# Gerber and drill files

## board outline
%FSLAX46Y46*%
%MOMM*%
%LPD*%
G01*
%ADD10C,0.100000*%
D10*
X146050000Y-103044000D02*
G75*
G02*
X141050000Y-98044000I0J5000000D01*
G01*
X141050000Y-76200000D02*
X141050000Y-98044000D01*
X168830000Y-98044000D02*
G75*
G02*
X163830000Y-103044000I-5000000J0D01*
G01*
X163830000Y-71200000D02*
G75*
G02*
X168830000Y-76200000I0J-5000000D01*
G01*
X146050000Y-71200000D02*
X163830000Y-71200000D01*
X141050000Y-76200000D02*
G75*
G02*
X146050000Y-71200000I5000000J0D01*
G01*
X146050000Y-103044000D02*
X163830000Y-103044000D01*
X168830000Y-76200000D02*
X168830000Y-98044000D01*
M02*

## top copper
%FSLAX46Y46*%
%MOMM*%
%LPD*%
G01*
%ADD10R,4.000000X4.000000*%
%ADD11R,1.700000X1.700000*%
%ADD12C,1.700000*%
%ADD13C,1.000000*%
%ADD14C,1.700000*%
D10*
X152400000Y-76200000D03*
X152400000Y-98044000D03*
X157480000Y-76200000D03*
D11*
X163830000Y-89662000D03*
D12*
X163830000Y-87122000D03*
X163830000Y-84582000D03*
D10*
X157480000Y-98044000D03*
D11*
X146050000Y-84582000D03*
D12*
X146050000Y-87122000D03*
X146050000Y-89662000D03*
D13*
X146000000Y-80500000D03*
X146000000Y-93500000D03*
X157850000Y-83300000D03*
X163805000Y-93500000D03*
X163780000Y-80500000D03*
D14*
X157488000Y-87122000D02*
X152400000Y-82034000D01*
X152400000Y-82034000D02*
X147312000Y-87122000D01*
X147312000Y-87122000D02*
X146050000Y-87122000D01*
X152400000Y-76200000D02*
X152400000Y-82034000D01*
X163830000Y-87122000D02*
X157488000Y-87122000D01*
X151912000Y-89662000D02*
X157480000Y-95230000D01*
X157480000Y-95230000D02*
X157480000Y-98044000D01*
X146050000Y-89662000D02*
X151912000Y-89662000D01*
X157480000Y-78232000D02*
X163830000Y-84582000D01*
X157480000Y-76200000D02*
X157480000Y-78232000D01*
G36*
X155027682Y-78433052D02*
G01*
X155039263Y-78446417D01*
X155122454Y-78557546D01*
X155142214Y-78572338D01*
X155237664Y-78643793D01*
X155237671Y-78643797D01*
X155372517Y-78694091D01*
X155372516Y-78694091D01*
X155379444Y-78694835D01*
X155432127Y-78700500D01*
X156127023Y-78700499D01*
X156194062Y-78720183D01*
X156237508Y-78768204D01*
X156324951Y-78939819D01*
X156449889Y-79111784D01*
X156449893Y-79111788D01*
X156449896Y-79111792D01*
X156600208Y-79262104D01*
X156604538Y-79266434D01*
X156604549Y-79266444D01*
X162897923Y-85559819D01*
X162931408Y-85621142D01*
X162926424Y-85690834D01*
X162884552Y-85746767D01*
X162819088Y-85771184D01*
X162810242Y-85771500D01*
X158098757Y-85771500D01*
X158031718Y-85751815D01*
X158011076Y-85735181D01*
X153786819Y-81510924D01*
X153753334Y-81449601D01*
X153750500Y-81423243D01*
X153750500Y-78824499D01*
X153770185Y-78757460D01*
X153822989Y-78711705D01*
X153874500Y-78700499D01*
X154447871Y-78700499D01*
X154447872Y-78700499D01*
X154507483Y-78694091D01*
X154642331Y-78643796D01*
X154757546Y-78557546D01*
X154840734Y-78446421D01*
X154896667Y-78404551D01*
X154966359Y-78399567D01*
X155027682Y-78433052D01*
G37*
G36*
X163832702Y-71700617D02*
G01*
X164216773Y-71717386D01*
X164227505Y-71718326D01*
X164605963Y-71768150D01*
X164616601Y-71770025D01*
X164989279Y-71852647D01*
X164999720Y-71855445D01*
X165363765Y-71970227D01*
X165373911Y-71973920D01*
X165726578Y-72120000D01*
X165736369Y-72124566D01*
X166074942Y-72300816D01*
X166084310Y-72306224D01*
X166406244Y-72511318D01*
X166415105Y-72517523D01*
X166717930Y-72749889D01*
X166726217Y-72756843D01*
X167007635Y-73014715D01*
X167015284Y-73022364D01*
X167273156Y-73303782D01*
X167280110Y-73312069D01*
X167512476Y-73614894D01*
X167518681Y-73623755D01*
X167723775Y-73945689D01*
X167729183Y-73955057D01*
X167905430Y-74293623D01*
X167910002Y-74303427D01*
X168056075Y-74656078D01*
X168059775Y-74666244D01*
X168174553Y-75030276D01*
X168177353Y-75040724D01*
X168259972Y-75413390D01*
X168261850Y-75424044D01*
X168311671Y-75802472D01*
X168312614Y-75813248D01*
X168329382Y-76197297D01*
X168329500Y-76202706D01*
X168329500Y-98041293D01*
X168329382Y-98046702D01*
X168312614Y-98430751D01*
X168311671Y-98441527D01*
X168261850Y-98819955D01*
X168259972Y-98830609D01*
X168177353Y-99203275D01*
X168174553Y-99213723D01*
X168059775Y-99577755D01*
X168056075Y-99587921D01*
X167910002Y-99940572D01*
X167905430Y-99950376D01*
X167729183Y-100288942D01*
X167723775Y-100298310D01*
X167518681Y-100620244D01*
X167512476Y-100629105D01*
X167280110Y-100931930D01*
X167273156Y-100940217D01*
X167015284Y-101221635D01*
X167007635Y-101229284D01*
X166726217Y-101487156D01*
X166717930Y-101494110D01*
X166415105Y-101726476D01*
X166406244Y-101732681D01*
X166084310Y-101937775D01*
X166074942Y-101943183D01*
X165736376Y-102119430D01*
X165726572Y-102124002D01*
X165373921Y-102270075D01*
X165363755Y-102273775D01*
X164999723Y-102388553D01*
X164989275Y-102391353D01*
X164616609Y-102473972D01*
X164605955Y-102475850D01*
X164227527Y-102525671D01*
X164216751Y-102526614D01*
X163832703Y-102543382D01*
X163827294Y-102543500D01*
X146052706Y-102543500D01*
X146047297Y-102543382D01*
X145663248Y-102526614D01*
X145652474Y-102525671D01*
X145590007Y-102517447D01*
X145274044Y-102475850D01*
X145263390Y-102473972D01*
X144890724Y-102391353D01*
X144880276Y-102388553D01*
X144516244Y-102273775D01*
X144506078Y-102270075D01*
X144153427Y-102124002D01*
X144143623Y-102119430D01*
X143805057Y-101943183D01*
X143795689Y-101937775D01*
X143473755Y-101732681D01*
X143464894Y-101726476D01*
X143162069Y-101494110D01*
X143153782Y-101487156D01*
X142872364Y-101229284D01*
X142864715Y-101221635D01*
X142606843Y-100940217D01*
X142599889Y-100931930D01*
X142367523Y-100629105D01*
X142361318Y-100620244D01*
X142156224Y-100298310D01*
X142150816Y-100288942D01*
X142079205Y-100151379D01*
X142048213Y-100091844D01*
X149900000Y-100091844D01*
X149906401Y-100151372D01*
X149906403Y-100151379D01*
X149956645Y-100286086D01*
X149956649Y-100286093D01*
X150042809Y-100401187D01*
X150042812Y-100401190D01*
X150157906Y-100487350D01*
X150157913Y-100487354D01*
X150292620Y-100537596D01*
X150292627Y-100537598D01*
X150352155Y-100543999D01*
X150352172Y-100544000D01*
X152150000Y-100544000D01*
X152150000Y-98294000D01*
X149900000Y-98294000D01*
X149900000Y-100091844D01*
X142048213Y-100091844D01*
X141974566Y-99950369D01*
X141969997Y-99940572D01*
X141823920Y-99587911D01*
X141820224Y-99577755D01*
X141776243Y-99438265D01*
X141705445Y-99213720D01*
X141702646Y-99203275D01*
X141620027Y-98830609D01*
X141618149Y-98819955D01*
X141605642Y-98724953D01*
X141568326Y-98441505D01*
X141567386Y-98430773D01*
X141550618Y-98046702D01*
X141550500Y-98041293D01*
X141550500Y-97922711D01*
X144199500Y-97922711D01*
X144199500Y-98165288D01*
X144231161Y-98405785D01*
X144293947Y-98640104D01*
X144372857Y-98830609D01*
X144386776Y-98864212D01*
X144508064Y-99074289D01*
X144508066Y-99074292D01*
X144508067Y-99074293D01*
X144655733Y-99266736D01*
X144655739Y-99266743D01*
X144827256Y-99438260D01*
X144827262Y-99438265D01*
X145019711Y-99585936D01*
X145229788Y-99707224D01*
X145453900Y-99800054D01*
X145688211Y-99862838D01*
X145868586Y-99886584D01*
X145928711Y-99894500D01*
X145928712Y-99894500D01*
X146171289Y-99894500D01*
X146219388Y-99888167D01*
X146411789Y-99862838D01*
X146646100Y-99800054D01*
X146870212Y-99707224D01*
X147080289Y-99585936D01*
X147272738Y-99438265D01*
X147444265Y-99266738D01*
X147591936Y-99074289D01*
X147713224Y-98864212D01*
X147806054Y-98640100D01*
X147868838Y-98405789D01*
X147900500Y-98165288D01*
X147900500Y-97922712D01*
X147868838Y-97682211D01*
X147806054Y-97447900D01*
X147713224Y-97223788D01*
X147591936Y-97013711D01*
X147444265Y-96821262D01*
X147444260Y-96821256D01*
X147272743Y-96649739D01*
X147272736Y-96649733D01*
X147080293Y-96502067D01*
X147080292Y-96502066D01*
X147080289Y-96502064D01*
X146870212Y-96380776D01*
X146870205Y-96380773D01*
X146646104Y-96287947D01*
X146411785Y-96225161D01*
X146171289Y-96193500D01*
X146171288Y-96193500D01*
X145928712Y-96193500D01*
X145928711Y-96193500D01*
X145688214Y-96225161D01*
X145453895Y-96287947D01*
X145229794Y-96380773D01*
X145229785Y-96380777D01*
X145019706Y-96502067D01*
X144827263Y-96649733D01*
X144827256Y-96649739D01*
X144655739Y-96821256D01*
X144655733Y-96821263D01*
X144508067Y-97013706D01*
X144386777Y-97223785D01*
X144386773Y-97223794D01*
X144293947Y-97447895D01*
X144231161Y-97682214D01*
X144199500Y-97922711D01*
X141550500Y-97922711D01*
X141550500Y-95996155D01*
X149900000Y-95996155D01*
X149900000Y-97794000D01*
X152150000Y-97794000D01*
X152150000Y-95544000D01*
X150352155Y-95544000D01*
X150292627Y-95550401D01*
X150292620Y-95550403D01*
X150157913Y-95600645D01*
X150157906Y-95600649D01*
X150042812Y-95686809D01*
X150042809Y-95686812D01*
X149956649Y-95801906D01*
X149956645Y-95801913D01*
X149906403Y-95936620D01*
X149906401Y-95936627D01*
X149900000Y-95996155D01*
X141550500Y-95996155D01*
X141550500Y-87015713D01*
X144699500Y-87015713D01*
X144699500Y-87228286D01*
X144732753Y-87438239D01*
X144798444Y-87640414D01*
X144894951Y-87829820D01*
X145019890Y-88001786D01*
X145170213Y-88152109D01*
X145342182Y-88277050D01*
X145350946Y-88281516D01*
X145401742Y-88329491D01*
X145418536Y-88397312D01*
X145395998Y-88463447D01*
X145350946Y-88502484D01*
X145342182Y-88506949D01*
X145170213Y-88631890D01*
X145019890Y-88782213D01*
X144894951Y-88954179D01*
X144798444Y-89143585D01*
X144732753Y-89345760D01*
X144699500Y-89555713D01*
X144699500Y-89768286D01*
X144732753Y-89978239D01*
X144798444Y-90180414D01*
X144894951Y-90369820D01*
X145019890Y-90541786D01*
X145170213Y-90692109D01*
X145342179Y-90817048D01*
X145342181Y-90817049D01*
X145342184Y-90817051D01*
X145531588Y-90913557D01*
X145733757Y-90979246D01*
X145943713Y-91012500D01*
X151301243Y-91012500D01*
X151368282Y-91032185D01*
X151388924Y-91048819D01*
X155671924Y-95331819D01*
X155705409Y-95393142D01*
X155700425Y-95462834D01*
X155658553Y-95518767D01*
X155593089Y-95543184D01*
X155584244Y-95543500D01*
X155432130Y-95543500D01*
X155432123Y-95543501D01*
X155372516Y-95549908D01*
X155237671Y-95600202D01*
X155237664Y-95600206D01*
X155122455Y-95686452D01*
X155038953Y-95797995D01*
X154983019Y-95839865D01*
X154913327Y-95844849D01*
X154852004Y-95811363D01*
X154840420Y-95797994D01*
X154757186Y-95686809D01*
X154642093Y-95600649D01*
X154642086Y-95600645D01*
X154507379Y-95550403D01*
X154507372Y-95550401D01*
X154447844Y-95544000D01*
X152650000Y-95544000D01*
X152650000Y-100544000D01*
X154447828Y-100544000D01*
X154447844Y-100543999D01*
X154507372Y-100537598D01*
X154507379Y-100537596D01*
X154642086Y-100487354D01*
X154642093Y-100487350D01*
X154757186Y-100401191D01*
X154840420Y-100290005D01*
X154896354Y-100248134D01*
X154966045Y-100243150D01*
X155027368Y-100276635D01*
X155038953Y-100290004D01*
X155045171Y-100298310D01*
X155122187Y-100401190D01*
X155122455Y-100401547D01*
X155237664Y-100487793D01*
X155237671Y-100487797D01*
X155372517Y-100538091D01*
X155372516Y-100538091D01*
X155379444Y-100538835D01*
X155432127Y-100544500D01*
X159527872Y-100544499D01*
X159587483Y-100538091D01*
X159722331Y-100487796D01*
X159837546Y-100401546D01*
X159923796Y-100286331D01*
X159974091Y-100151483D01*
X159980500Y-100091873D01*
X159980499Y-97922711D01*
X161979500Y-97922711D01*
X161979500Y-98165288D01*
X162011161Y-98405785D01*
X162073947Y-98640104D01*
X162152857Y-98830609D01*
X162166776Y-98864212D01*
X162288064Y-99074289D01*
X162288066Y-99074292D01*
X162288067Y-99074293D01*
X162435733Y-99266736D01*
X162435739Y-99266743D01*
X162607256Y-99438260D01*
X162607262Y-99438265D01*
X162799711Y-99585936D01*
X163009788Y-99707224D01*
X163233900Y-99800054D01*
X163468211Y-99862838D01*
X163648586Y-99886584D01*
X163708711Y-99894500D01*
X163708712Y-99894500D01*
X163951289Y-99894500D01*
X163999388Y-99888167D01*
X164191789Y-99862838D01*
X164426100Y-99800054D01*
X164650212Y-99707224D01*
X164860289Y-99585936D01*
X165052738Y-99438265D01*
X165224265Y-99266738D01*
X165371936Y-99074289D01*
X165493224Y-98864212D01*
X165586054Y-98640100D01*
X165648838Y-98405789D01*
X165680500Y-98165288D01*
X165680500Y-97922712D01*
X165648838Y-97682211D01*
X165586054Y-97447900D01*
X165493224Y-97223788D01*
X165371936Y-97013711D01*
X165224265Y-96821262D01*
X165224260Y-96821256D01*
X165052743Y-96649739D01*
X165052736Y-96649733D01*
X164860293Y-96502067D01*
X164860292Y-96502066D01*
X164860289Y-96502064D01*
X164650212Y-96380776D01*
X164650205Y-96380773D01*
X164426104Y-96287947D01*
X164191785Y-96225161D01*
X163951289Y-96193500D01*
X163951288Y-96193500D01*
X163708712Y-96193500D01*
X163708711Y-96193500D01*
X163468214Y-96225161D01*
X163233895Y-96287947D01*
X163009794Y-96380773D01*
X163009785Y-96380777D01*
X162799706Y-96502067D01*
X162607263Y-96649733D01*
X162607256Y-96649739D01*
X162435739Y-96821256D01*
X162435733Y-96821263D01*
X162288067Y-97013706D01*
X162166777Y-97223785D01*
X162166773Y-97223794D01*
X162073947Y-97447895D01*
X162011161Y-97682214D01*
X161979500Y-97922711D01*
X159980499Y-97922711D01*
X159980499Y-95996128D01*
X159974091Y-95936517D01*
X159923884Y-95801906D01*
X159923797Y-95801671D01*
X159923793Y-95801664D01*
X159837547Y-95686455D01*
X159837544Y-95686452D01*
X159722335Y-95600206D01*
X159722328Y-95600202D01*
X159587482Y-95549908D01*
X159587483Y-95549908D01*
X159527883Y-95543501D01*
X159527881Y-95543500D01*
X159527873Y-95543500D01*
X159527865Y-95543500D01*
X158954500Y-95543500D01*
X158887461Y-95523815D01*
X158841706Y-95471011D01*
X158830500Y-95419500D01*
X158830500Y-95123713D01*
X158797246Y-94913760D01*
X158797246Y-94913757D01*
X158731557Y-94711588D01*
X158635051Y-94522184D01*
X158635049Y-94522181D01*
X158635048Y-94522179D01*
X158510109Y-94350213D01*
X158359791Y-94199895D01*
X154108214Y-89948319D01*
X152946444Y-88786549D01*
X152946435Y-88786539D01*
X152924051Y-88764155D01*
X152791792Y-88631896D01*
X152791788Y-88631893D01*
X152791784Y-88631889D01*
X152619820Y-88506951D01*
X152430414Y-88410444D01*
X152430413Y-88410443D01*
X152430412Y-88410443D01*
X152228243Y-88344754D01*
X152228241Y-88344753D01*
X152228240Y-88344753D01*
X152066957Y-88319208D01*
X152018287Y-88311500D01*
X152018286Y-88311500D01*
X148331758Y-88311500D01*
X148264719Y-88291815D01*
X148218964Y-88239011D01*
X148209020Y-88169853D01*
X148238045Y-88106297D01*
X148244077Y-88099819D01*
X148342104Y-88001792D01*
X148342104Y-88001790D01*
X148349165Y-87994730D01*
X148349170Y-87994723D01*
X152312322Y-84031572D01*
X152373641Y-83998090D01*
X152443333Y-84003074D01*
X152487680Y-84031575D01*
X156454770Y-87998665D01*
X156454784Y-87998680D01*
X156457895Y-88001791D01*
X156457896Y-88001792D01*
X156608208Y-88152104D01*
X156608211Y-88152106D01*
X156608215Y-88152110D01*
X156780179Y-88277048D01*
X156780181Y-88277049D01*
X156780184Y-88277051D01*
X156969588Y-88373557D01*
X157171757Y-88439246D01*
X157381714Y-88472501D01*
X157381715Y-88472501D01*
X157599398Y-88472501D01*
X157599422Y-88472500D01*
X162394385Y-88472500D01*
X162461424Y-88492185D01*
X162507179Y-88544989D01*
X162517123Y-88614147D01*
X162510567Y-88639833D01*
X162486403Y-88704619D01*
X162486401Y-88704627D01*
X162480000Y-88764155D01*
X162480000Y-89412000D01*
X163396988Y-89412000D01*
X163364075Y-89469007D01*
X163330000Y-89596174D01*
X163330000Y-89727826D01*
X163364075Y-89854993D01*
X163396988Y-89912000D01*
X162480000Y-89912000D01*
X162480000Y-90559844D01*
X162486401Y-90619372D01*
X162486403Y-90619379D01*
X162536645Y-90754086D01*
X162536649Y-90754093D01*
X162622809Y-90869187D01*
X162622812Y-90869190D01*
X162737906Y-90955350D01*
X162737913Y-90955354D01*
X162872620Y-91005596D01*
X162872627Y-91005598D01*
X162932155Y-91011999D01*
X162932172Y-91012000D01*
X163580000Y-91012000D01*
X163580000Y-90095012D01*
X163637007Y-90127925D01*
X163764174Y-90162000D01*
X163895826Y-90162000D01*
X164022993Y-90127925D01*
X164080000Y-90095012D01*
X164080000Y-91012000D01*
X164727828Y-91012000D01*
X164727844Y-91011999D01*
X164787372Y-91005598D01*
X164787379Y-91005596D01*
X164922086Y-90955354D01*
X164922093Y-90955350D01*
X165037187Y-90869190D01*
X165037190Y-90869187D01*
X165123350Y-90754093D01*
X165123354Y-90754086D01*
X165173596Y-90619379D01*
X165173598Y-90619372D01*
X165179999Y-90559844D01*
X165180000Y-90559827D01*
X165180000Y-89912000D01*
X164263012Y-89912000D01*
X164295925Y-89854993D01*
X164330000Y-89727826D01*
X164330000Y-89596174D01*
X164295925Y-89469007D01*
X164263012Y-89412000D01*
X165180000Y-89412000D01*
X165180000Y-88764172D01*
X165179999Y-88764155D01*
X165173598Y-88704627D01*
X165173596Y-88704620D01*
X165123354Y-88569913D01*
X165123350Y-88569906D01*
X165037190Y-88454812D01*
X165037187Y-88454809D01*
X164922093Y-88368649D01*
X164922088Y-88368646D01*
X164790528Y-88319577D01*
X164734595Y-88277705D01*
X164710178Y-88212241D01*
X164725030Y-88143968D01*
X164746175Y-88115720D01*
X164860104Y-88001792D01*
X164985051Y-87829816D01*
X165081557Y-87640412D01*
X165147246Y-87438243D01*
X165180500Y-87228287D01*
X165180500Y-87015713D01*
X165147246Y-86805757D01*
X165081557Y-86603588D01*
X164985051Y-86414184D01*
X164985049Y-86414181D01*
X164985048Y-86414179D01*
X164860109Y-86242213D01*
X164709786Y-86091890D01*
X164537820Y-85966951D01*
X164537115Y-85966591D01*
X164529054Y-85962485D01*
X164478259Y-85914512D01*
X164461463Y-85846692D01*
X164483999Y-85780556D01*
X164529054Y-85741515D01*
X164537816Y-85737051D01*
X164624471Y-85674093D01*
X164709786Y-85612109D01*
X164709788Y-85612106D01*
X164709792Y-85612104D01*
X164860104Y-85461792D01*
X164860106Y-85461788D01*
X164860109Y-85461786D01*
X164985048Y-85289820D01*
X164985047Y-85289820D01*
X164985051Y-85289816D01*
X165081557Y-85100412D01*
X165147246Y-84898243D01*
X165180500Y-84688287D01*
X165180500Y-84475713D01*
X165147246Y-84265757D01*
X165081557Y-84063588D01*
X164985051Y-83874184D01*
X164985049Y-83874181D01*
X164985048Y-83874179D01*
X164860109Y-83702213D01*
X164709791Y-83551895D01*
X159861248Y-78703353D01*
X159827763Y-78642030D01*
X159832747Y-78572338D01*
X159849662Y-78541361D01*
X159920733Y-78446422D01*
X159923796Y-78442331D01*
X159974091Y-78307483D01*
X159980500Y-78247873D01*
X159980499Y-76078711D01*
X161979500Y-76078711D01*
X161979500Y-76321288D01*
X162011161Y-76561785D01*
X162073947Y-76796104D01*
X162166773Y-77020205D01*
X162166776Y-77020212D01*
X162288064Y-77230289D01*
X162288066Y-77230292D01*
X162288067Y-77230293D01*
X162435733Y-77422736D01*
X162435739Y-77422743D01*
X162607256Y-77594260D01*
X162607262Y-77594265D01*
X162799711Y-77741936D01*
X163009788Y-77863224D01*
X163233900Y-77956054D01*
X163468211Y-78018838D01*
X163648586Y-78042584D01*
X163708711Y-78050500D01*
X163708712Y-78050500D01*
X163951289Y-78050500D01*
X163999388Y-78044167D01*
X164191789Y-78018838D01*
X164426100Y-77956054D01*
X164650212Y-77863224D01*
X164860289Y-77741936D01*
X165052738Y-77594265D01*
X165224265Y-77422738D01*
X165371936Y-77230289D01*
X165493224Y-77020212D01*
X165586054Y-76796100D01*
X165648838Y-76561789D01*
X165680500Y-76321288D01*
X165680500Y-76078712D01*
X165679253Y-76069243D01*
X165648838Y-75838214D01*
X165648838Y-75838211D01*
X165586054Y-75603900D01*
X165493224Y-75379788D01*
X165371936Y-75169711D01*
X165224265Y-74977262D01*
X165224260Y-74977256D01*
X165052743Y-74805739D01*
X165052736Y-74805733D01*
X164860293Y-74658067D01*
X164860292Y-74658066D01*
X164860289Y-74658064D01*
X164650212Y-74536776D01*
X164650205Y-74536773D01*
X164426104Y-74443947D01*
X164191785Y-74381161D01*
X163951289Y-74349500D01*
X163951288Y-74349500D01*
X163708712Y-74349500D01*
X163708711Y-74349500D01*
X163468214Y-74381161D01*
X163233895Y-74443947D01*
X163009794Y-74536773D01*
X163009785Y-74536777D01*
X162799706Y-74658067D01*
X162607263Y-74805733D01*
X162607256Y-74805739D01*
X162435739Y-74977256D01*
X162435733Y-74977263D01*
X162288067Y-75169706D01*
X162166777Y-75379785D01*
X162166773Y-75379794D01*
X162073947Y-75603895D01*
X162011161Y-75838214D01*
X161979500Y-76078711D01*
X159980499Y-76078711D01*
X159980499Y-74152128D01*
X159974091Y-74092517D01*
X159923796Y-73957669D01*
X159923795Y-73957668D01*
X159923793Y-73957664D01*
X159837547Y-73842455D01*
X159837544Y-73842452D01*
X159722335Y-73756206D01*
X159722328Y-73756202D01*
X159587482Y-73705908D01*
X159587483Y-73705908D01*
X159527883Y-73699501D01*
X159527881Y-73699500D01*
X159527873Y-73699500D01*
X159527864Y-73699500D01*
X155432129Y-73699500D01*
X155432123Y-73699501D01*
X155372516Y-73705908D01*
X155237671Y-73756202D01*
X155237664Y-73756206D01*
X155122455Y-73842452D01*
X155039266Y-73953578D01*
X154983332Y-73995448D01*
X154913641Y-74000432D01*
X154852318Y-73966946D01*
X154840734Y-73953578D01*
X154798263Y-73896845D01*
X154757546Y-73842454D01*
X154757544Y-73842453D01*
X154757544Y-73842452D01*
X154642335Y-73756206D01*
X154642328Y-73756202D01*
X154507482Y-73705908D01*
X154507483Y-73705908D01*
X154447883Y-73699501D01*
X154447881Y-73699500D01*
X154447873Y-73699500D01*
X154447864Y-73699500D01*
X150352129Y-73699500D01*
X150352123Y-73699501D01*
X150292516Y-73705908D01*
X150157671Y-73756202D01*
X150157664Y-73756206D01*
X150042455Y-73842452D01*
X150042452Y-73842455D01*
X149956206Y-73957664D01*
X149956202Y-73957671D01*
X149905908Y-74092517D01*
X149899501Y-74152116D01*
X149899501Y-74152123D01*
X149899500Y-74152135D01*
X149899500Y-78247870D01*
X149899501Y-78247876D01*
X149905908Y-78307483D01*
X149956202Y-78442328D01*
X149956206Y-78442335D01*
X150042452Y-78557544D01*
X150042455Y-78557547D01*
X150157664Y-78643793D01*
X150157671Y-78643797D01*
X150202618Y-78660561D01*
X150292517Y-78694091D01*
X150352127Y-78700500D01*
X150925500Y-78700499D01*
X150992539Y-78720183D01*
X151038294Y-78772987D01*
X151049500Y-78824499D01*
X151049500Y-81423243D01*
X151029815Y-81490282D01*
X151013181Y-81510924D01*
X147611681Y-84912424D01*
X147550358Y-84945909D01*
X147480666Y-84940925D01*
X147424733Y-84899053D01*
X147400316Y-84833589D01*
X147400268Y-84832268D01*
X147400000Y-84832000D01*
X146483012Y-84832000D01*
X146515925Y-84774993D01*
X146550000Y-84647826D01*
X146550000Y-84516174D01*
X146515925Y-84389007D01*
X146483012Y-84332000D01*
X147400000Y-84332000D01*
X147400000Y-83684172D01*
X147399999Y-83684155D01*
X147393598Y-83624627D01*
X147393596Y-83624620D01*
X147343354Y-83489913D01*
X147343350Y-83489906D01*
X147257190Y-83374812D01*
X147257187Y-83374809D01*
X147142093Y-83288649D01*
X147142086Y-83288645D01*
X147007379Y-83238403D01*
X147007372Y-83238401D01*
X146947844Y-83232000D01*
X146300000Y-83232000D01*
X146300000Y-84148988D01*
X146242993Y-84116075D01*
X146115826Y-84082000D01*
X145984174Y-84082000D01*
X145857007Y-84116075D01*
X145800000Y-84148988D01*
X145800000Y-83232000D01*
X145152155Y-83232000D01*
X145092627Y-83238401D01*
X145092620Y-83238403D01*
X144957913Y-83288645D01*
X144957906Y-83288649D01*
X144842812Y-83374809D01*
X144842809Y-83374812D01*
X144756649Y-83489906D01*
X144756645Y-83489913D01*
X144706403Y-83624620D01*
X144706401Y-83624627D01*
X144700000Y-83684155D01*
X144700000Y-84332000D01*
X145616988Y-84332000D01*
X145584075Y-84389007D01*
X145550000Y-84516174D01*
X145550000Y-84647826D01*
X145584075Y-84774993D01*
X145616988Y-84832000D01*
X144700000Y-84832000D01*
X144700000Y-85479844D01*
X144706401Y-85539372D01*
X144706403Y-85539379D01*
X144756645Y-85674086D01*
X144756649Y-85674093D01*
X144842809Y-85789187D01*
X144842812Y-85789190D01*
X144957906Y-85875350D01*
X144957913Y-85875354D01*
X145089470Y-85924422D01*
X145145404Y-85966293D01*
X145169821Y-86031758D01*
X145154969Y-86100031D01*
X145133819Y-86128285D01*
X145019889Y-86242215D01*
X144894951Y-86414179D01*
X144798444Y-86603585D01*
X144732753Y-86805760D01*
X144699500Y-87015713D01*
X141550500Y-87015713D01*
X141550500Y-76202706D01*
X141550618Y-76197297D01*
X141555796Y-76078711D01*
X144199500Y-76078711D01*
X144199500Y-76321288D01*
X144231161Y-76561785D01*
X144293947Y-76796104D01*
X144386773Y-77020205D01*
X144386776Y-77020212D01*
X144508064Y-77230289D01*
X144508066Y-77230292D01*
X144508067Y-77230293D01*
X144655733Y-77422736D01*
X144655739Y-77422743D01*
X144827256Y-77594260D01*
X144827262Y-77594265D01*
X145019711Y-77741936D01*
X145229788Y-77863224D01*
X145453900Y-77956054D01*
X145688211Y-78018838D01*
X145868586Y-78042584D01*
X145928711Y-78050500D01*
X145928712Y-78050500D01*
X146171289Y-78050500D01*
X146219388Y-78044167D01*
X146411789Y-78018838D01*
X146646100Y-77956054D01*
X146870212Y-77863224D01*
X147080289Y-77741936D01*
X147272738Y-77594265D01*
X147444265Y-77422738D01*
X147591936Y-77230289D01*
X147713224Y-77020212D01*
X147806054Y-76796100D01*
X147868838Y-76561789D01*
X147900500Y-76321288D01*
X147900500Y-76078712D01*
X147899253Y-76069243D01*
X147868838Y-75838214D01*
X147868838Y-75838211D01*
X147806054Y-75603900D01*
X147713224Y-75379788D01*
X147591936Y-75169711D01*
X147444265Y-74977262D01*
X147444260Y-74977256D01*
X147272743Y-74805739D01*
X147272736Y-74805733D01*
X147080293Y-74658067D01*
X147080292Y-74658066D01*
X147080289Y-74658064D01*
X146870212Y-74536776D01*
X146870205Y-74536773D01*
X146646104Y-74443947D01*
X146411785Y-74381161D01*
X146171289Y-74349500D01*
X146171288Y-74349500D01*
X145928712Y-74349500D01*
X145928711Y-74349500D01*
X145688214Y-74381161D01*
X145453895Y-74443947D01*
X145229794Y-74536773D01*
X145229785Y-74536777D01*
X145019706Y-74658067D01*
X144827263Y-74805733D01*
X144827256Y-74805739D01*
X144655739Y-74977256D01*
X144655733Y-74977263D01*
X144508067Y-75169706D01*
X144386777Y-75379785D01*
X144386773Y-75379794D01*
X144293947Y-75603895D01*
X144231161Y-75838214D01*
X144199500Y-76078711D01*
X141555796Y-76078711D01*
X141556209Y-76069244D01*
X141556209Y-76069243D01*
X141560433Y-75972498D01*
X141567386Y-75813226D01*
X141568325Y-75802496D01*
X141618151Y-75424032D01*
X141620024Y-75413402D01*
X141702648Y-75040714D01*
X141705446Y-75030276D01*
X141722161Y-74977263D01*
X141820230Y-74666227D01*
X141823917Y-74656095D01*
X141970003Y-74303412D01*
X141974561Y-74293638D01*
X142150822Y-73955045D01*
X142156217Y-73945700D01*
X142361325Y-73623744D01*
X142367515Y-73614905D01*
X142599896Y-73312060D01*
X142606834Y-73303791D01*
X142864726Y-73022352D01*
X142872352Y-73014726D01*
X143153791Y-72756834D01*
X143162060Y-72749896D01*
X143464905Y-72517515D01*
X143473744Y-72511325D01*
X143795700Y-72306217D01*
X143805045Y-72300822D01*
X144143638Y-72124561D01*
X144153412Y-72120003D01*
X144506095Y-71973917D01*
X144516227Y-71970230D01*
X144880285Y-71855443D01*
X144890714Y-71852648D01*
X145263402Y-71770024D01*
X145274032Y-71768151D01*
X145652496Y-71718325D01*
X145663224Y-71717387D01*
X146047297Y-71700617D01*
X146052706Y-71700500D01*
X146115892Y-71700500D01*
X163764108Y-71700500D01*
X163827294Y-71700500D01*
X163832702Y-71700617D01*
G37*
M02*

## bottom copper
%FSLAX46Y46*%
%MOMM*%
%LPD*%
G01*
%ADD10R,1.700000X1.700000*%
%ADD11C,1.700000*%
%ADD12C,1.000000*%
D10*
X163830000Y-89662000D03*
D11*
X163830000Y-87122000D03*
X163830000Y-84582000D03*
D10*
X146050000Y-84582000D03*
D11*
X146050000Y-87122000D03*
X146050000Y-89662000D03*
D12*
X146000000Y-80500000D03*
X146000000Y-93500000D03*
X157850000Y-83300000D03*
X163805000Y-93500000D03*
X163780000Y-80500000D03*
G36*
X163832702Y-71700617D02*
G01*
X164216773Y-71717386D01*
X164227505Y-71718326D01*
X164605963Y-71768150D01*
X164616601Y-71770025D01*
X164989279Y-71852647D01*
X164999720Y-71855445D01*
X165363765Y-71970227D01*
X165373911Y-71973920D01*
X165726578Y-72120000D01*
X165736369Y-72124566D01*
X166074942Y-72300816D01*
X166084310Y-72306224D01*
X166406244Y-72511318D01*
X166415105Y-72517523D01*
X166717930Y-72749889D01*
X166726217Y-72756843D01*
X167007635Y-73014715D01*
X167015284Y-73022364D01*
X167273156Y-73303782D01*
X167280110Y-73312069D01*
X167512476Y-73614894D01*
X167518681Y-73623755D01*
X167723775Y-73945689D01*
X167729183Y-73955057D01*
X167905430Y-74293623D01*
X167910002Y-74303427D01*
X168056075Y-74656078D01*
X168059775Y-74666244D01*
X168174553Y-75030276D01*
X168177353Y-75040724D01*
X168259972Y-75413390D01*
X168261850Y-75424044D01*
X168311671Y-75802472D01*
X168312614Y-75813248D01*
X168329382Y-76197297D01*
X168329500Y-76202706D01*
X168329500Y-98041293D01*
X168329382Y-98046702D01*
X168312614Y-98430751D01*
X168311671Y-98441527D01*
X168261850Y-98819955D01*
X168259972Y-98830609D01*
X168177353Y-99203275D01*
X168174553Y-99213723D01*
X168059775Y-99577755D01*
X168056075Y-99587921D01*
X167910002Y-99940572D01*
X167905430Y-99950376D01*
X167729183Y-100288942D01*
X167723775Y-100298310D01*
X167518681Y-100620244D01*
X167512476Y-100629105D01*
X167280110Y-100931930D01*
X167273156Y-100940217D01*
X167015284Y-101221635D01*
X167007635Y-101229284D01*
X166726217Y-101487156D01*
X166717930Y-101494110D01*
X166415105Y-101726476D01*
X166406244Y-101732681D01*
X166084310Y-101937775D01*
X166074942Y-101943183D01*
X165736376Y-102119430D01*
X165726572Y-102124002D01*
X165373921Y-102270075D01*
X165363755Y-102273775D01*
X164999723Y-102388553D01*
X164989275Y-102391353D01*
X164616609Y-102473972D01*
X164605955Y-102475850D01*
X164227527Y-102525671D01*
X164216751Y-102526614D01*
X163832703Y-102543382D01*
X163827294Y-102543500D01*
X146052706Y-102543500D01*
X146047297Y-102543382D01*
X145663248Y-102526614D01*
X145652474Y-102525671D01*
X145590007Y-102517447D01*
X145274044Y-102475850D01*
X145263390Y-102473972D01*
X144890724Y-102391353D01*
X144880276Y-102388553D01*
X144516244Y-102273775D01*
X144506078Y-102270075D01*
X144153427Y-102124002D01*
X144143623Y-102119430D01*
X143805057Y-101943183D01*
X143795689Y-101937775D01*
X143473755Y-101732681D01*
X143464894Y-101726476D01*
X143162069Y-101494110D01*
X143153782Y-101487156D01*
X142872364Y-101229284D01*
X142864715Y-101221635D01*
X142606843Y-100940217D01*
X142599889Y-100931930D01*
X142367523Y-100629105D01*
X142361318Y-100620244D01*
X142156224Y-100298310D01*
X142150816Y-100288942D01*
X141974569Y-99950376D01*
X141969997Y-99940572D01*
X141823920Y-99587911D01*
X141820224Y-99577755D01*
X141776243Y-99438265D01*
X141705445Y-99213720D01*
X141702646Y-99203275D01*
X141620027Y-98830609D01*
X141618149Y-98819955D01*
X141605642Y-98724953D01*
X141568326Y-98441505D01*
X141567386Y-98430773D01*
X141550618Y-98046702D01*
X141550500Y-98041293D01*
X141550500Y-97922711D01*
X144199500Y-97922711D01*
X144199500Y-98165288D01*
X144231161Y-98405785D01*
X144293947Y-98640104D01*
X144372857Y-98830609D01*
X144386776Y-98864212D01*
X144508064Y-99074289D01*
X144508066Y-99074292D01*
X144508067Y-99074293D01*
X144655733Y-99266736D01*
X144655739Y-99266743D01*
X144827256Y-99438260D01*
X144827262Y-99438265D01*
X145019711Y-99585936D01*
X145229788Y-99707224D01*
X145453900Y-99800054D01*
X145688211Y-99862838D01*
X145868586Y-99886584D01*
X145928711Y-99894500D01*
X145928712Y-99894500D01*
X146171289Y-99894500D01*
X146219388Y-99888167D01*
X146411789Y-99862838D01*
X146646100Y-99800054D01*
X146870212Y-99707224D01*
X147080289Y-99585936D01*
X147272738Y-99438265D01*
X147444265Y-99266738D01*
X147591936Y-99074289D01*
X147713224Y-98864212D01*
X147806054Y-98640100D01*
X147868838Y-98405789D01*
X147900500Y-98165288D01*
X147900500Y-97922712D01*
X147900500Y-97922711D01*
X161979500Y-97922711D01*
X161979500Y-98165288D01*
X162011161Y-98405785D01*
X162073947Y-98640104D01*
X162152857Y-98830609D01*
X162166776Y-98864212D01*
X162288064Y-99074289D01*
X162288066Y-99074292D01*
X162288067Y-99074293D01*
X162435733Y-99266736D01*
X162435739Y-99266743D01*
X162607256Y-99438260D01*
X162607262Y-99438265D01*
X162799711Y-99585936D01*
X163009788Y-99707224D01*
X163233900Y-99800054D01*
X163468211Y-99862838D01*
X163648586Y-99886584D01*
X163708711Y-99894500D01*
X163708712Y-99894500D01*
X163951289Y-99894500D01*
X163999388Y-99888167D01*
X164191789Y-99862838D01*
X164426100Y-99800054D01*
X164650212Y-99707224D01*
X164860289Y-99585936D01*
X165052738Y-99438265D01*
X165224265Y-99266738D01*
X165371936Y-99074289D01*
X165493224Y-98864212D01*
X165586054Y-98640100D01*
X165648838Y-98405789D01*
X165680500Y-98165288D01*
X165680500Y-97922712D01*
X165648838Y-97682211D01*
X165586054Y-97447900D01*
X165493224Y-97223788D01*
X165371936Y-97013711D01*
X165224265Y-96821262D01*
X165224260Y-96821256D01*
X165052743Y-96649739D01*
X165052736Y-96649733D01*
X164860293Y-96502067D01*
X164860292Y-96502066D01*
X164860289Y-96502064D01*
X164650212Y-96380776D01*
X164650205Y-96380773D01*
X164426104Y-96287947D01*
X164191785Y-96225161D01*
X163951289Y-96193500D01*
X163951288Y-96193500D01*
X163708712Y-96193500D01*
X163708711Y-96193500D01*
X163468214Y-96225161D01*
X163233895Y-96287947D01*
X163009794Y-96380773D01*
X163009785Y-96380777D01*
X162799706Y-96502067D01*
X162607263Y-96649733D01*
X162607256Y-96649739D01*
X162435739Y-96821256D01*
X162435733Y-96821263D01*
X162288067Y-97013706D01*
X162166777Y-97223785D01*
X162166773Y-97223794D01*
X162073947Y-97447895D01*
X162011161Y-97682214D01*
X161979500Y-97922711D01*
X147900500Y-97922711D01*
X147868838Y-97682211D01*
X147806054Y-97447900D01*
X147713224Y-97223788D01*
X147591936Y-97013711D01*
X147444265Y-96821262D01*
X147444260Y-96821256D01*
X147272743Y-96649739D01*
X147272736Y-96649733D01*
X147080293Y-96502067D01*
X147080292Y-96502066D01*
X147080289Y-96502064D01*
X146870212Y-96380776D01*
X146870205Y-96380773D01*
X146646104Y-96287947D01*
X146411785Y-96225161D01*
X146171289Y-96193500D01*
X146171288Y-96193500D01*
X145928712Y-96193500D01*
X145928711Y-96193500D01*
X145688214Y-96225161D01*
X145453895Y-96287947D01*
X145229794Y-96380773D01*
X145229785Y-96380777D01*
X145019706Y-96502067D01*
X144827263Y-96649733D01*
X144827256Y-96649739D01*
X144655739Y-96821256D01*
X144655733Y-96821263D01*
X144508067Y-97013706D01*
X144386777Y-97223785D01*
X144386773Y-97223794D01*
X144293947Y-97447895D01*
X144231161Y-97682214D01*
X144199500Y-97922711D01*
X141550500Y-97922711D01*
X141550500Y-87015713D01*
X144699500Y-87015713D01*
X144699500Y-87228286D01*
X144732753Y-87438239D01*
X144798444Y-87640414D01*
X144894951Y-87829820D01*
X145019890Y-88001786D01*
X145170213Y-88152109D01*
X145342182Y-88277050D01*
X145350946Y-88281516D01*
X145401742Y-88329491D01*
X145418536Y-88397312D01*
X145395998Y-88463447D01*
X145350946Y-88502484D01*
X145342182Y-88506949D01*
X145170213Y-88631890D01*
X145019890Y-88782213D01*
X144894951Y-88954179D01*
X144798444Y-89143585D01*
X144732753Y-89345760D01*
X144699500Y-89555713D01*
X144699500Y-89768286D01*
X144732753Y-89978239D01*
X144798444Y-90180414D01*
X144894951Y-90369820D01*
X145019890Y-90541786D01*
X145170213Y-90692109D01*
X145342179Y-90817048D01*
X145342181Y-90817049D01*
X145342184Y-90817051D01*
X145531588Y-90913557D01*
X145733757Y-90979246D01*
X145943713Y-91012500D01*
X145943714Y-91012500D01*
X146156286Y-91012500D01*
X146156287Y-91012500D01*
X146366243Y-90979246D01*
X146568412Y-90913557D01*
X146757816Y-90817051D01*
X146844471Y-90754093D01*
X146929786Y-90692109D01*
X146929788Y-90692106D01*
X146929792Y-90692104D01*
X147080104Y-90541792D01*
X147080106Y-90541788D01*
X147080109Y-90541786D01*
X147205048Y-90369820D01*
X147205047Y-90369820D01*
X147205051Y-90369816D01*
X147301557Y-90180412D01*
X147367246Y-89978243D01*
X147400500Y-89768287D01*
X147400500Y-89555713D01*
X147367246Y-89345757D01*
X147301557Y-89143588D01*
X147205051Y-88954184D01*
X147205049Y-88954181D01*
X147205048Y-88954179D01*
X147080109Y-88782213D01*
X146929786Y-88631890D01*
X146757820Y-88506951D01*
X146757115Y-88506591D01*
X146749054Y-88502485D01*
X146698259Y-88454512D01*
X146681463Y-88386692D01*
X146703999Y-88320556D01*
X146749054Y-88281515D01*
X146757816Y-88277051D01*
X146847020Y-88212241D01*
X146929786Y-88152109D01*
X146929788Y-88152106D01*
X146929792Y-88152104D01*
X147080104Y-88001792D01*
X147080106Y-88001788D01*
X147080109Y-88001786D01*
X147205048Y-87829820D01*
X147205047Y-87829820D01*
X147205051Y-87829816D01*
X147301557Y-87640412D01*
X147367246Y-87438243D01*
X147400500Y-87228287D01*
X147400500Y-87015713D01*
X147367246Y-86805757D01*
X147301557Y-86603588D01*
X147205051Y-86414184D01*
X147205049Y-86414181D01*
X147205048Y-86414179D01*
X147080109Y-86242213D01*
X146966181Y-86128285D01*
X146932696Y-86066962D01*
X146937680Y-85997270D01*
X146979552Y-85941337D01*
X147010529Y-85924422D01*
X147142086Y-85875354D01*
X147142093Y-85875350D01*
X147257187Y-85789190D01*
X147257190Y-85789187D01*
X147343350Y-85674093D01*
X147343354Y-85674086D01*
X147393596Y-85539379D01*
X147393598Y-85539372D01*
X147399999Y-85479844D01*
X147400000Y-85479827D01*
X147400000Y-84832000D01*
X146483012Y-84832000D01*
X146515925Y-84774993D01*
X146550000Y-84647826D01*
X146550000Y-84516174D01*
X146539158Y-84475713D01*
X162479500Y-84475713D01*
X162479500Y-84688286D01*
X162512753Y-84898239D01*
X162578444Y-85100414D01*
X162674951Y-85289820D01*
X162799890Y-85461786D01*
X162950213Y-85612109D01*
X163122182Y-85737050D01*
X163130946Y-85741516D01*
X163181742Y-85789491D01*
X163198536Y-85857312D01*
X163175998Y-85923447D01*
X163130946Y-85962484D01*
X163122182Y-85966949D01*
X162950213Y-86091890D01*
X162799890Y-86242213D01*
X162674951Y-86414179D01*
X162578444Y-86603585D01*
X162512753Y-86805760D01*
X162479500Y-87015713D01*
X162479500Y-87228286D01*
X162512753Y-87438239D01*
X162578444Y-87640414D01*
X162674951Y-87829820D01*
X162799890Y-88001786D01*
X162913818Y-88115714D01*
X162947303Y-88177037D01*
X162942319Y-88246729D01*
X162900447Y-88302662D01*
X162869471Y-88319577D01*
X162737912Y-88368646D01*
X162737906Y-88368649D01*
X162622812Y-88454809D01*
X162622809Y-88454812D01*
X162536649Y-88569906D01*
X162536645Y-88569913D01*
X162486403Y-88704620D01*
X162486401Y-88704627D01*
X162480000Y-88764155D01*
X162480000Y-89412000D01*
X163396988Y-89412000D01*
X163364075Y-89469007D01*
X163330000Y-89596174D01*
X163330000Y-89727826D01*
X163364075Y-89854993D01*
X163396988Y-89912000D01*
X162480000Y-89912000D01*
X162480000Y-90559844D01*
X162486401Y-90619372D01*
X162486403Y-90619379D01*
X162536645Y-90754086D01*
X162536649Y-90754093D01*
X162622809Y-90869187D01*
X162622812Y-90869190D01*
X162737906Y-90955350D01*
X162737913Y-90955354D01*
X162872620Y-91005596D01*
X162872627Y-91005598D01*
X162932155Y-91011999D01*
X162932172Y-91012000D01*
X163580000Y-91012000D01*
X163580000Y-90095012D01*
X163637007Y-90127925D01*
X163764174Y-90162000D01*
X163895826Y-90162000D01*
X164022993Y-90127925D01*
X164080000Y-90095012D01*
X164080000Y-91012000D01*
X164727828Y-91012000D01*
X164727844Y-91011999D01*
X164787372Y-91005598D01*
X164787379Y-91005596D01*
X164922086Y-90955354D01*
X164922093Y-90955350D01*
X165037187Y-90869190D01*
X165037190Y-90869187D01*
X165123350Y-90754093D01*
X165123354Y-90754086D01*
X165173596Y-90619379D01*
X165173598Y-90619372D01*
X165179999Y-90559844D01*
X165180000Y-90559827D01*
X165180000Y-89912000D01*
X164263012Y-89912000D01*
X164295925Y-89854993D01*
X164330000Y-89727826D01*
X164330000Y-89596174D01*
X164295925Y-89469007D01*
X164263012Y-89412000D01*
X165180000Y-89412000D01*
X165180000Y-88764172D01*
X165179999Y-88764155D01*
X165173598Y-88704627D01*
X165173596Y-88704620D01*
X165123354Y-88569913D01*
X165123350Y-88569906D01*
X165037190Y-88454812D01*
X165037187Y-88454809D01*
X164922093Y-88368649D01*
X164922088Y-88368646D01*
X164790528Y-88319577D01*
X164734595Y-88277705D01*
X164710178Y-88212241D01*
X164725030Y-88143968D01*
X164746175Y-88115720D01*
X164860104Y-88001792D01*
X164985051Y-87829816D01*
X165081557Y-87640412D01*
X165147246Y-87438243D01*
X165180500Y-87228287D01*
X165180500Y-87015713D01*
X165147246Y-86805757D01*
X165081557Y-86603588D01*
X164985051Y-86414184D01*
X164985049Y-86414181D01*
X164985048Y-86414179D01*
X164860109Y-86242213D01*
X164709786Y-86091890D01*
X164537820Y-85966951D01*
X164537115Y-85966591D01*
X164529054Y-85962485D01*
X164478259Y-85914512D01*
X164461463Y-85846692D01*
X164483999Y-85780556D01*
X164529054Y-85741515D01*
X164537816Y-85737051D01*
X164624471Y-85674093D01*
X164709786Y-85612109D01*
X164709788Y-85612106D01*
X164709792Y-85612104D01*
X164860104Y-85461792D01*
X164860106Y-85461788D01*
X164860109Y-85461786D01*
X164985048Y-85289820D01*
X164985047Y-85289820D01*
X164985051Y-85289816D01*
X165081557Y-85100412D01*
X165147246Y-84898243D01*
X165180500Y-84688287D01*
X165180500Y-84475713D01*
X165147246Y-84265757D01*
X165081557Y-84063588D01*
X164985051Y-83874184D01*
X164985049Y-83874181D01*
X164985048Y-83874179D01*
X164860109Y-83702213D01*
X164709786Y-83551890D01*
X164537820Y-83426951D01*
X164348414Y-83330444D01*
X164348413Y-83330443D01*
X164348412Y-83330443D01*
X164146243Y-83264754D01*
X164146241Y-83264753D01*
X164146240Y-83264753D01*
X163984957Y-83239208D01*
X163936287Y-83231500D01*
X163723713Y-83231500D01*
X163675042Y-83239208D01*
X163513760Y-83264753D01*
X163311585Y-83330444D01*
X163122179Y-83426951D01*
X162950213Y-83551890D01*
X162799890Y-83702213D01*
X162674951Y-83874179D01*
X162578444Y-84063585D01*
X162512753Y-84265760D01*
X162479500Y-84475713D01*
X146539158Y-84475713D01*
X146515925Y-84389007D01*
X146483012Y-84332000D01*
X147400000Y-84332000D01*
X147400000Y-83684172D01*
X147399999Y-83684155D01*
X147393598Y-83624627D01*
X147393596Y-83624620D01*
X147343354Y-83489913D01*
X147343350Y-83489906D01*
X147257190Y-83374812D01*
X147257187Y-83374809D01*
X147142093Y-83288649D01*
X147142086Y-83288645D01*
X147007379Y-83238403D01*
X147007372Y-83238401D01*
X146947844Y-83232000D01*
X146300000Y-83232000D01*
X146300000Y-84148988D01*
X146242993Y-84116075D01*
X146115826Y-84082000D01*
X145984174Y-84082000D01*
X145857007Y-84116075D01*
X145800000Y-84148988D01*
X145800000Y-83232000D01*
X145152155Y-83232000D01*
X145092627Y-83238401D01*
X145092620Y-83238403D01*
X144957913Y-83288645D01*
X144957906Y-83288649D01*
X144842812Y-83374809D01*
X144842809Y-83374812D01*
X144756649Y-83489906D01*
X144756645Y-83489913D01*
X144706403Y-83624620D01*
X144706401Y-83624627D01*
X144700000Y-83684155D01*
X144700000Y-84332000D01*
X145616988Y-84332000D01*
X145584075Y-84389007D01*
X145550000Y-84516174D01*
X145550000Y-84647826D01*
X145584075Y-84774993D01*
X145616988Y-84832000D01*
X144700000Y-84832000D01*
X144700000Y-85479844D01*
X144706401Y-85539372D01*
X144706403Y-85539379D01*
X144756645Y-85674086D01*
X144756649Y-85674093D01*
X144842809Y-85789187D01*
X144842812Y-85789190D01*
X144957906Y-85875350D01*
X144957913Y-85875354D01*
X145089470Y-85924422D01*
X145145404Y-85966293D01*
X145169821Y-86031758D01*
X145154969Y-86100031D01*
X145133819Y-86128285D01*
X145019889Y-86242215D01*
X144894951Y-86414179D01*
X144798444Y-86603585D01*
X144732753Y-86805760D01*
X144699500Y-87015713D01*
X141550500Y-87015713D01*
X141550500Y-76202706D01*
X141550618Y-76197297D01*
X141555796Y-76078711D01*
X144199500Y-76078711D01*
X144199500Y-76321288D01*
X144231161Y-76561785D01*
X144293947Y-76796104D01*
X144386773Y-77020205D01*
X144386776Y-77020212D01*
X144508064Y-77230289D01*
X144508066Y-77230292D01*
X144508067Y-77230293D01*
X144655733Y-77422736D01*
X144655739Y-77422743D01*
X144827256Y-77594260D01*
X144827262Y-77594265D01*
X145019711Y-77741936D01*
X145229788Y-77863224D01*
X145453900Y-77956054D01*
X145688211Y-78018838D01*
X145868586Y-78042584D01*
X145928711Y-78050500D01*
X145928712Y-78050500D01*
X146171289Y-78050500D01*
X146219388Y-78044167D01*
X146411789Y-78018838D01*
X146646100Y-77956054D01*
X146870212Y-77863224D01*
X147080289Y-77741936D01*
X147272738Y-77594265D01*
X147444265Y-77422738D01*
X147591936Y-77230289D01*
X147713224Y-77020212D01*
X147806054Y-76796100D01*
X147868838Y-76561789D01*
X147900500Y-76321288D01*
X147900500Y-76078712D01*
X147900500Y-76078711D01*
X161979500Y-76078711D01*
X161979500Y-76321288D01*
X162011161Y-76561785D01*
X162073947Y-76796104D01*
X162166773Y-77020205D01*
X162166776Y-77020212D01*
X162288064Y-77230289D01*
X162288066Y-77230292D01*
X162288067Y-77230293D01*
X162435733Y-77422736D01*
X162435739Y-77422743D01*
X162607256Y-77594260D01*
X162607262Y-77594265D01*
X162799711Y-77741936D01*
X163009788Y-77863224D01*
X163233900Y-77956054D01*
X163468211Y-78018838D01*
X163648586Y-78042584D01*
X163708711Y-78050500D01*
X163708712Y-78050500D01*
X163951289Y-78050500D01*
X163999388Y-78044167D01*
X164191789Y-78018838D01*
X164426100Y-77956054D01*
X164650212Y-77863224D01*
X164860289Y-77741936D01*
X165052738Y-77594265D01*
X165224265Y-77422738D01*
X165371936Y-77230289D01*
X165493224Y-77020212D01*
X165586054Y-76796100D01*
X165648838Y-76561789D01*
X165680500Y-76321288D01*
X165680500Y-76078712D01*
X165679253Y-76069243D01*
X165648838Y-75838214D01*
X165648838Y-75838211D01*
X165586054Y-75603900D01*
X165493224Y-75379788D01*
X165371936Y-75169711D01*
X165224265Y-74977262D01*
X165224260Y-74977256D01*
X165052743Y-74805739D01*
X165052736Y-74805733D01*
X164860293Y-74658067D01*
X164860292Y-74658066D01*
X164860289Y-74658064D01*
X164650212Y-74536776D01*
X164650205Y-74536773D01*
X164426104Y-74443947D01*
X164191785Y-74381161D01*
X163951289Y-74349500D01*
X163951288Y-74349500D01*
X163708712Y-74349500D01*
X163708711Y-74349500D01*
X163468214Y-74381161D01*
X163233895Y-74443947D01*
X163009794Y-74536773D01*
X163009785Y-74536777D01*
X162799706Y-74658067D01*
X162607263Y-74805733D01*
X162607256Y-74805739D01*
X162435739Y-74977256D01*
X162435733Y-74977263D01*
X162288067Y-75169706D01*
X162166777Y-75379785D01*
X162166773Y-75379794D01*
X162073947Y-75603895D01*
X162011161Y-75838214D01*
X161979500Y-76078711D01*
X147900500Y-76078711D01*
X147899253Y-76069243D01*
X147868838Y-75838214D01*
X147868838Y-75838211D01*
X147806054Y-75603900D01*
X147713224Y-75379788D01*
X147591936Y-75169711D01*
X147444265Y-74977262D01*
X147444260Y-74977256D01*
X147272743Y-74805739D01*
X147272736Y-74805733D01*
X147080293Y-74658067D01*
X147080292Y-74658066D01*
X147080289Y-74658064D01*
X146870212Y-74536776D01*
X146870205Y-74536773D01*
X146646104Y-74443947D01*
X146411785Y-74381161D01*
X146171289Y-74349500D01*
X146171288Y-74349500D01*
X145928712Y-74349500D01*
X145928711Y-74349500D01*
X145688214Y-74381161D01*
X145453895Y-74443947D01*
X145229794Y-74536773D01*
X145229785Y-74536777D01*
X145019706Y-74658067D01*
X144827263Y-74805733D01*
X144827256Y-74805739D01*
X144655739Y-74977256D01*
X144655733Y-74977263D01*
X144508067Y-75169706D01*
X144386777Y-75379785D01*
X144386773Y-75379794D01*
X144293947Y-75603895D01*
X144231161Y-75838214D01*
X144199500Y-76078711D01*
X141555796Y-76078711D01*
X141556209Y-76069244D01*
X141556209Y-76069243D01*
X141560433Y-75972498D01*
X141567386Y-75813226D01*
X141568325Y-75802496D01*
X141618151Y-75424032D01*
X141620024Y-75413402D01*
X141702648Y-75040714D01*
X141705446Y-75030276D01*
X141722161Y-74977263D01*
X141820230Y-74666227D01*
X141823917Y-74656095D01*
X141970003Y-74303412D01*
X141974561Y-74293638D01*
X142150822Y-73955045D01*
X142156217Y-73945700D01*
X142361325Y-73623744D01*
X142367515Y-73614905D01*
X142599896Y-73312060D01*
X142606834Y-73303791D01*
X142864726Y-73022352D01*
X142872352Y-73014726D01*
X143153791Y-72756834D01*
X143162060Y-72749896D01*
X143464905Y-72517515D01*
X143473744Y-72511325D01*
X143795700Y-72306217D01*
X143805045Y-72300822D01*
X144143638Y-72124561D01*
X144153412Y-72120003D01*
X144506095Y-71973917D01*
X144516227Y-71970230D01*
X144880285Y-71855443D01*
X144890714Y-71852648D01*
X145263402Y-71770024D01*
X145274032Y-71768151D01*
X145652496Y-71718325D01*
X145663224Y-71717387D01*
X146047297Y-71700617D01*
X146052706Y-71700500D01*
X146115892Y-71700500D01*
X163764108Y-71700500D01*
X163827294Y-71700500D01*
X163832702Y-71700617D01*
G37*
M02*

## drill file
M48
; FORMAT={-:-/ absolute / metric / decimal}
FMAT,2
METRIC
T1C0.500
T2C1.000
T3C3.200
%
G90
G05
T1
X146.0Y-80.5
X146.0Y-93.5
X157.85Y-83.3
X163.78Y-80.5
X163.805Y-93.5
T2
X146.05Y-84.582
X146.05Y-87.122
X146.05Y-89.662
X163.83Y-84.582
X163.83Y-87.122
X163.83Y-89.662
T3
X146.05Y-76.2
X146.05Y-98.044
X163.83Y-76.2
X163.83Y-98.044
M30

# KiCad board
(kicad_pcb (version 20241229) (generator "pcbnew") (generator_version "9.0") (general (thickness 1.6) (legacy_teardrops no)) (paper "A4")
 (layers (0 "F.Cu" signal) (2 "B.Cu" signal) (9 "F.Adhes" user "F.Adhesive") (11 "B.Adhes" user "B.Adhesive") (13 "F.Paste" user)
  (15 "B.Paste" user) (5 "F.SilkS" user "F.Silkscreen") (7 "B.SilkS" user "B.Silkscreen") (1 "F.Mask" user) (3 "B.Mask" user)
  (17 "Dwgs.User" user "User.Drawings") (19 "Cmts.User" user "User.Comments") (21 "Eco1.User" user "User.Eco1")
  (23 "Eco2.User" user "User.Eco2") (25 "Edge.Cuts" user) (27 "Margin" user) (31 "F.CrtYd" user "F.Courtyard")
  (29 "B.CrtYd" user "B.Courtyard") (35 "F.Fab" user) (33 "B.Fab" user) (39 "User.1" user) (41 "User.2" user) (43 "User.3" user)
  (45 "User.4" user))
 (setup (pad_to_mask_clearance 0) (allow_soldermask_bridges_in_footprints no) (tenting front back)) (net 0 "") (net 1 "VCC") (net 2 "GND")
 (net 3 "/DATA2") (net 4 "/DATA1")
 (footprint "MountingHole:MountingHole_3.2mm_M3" (layer "F.Cu") (at 146.05 98.044)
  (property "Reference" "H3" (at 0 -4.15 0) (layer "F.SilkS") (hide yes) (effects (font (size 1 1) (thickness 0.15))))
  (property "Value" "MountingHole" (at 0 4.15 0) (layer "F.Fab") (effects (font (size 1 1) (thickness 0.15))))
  (pad "" np_thru_hole circle (at 0 0) (size 3.2 3.2) (drill 3.2) (layers "*.Cu" "*.Mask")))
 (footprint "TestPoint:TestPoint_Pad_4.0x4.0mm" (layer "F.Cu") (at 152.4 76.2)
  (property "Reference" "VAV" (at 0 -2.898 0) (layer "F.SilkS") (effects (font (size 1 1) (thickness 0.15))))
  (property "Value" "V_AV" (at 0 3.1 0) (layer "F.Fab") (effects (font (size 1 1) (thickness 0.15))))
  (pad "1" smd rect (at 0 0) (size 4 4) (layers "F.Cu" "F.Mask") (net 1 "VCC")))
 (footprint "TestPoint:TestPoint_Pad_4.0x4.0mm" (layer "F.Cu") (at 152.4 98.044)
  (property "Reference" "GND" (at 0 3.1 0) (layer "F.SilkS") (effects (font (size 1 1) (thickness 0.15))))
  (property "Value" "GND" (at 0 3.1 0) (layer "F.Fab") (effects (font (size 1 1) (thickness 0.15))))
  (pad "1" smd rect (at 0 0) (size 4 4) (layers "F.Cu" "F.Mask") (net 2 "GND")))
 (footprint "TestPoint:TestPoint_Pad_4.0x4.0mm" (layer "F.Cu") (at 157.48 76.2)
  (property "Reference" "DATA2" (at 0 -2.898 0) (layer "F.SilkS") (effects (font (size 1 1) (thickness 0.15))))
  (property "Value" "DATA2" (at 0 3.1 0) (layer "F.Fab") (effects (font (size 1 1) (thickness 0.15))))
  (pad "1" smd rect (at 0 0) (size 4 4) (layers "F.Cu" "F.Mask") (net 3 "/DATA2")))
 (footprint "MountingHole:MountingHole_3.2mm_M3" (layer "F.Cu") (at 146.05 76.2)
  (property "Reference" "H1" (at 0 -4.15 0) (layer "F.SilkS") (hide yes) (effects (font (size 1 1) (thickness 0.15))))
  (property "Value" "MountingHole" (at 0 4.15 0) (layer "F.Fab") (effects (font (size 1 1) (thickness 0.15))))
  (pad "" np_thru_hole circle (at 0 0) (size 3.2 3.2) (drill 3.2) (layers "*.Cu" "*.Mask")))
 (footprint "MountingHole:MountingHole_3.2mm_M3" (layer "F.Cu") (at 163.83 76.2)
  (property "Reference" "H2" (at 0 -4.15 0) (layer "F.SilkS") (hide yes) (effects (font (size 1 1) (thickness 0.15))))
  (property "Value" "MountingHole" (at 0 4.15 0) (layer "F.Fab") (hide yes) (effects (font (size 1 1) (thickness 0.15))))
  (pad "" np_thru_hole circle (at 0 0) (size 3.2 3.2) (drill 3.2) (layers "*.Cu" "*.Mask")))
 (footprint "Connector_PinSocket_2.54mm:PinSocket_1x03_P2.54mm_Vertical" (layer "F.Cu") (at 163.83 89.662 180)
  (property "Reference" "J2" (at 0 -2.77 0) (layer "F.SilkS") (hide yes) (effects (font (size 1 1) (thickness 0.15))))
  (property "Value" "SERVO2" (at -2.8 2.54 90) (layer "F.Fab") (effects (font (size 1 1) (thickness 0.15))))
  (pad "1" thru_hole rect (at 0 0 180) (size 1.7 1.7) (drill 1) (layers "*.Cu" "*.Mask") (remove_unused_layers no) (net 2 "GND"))
  (pad "2" thru_hole circle (at 0 2.54 180) (size 1.7 1.7) (drill 1) (layers "*.Cu" "*.Mask") (remove_unused_layers no) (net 1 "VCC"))
  (pad "3" thru_hole circle (at 0 5.08 180) (size 1.7 1.7) (drill 1) (layers "*.Cu" "*.Mask") (remove_unused_layers no) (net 3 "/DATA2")))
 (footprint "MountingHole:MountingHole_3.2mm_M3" (layer "F.Cu") (at 163.83 98.044)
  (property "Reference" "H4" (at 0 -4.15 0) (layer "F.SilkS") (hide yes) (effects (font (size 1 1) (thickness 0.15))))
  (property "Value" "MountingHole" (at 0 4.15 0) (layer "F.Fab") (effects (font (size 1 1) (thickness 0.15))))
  (pad "" np_thru_hole circle (at 0 0) (size 3.2 3.2) (drill 3.2) (layers "*.Cu" "*.Mask")))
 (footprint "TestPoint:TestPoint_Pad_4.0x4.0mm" (layer "F.Cu") (at 157.48 98.044)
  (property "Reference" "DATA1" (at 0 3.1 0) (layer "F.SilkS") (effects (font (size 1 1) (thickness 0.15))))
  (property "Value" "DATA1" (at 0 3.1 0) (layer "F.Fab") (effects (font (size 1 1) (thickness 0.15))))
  (pad "1" smd rect (at 0 0) (size 4 4) (layers "F.Cu" "F.Mask") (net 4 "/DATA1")))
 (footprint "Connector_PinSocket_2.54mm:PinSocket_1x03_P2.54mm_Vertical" (layer "F.Cu") (at 146.05 84.582)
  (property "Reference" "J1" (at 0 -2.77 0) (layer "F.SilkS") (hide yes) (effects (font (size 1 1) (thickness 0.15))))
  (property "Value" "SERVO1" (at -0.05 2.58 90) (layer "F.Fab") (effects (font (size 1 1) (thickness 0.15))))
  (pad "1" thru_hole rect (at 0 0) (size 1.7 1.7) (drill 1) (layers "*.Cu" "*.Mask") (remove_unused_layers no) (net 2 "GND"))
  (pad "2" thru_hole circle (at 0 2.54) (size 1.7 1.7) (drill 1) (layers "*.Cu" "*.Mask") (remove_unused_layers no) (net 1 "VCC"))
  (pad "3" thru_hole circle (at 0 5.08) (size 1.7 1.7) (drill 1) (layers "*.Cu" "*.Mask") (remove_unused_layers no) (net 4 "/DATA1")))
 (gr_arc (start 146.05 103.044) (mid 142.514466 101.579534) (end 141.05 98.044) (stroke (width 0.1) (type solid)) (layer "Edge.Cuts"))
 (gr_line (start 141.05 76.2) (end 141.05 98.044) (stroke (width 0.1) (type solid)) (layer "Edge.Cuts"))
 (gr_arc (start 168.83 98.044) (mid 167.365534 101.579534) (end 163.83 103.044) (stroke (width 0.1) (type solid)) (layer "Edge.Cuts"))
 (gr_arc (start 163.83 71.2) (mid 167.365534 72.664466) (end 168.83 76.2) (stroke (width 0.1) (type solid)) (layer "Edge.Cuts"))
 (gr_line (start 146.05 71.2) (end 163.83 71.2) (stroke (width 0.1) (type solid)) (layer "Edge.Cuts"))
 (gr_arc (start 141.05 76.2) (mid 142.514466 72.664466) (end 146.05 71.2) (stroke (width 0.1) (type solid)) (layer "Edge.Cuts"))
 (gr_line (start 146.05 103.044) (end 163.83 103.044) (stroke (width 0.1) (type solid)) (layer "Edge.Cuts"))
 (gr_line (start 168.83 76.2) (end 168.83 98.044) (stroke (width 0.1) (type solid)) (layer "Edge.Cuts"))
 (segment (start 157.488 87.122) (end 152.4 82.034) (width 1.7) (layer "F.Cu") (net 1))
 (segment (start 152.4 82.034) (end 147.312 87.122) (width 1.7) (layer "F.Cu") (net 1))
 (segment (start 147.312 87.122) (end 146.05 87.122) (width 1.7) (layer "F.Cu") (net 1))
 (segment (start 152.4 76.2) (end 152.4 82.034) (width 1.7) (layer "F.Cu") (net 1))
 (segment (start 163.83 87.122) (end 157.488 87.122) (width 1.7) (layer "F.Cu") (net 1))
 (via (at 146 80.5) (size 1) (drill 0.5) (layers "F.Cu" "B.Cu") (free yes) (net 2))
 (via (at 146 93.5) (size 1) (drill 0.5) (layers "F.Cu" "B.Cu") (free yes) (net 2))
 (via (at 157.85 83.3) (size 1) (drill 0.5) (layers "F.Cu" "B.Cu") (free yes) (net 2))
 (via (at 163.805 93.5) (size 1) (drill 0.5) (layers "F.Cu" "B.Cu") (free yes) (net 2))
 (via (at 163.78 80.5) (size 1) (drill 0.5) (layers "F.Cu" "B.Cu") (free yes) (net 2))
 (segment (start 151.912 89.662) (end 157.48 95.23) (width 1.7) (layer "F.Cu") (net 4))
 (segment (start 157.48 95.23) (end 157.48 98.044) (width 1.7) (layer "F.Cu") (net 4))
 (segment (start 146.05 89.662) (end 151.912 89.662) (width 1.7) (layer "F.Cu") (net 4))
 (segment (start 157.48 78.232) (end 163.83 84.582) (width 1.7) (layer "F.Cu") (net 3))
 (segment (start 157.48 76.2) (end 157.48 78.232) (width 1.7) (layer "F.Cu") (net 3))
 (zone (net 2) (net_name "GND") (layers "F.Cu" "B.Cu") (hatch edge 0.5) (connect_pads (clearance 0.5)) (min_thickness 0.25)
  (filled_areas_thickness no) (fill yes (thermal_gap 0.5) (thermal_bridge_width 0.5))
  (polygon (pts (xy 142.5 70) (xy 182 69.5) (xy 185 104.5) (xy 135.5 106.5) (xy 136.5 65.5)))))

